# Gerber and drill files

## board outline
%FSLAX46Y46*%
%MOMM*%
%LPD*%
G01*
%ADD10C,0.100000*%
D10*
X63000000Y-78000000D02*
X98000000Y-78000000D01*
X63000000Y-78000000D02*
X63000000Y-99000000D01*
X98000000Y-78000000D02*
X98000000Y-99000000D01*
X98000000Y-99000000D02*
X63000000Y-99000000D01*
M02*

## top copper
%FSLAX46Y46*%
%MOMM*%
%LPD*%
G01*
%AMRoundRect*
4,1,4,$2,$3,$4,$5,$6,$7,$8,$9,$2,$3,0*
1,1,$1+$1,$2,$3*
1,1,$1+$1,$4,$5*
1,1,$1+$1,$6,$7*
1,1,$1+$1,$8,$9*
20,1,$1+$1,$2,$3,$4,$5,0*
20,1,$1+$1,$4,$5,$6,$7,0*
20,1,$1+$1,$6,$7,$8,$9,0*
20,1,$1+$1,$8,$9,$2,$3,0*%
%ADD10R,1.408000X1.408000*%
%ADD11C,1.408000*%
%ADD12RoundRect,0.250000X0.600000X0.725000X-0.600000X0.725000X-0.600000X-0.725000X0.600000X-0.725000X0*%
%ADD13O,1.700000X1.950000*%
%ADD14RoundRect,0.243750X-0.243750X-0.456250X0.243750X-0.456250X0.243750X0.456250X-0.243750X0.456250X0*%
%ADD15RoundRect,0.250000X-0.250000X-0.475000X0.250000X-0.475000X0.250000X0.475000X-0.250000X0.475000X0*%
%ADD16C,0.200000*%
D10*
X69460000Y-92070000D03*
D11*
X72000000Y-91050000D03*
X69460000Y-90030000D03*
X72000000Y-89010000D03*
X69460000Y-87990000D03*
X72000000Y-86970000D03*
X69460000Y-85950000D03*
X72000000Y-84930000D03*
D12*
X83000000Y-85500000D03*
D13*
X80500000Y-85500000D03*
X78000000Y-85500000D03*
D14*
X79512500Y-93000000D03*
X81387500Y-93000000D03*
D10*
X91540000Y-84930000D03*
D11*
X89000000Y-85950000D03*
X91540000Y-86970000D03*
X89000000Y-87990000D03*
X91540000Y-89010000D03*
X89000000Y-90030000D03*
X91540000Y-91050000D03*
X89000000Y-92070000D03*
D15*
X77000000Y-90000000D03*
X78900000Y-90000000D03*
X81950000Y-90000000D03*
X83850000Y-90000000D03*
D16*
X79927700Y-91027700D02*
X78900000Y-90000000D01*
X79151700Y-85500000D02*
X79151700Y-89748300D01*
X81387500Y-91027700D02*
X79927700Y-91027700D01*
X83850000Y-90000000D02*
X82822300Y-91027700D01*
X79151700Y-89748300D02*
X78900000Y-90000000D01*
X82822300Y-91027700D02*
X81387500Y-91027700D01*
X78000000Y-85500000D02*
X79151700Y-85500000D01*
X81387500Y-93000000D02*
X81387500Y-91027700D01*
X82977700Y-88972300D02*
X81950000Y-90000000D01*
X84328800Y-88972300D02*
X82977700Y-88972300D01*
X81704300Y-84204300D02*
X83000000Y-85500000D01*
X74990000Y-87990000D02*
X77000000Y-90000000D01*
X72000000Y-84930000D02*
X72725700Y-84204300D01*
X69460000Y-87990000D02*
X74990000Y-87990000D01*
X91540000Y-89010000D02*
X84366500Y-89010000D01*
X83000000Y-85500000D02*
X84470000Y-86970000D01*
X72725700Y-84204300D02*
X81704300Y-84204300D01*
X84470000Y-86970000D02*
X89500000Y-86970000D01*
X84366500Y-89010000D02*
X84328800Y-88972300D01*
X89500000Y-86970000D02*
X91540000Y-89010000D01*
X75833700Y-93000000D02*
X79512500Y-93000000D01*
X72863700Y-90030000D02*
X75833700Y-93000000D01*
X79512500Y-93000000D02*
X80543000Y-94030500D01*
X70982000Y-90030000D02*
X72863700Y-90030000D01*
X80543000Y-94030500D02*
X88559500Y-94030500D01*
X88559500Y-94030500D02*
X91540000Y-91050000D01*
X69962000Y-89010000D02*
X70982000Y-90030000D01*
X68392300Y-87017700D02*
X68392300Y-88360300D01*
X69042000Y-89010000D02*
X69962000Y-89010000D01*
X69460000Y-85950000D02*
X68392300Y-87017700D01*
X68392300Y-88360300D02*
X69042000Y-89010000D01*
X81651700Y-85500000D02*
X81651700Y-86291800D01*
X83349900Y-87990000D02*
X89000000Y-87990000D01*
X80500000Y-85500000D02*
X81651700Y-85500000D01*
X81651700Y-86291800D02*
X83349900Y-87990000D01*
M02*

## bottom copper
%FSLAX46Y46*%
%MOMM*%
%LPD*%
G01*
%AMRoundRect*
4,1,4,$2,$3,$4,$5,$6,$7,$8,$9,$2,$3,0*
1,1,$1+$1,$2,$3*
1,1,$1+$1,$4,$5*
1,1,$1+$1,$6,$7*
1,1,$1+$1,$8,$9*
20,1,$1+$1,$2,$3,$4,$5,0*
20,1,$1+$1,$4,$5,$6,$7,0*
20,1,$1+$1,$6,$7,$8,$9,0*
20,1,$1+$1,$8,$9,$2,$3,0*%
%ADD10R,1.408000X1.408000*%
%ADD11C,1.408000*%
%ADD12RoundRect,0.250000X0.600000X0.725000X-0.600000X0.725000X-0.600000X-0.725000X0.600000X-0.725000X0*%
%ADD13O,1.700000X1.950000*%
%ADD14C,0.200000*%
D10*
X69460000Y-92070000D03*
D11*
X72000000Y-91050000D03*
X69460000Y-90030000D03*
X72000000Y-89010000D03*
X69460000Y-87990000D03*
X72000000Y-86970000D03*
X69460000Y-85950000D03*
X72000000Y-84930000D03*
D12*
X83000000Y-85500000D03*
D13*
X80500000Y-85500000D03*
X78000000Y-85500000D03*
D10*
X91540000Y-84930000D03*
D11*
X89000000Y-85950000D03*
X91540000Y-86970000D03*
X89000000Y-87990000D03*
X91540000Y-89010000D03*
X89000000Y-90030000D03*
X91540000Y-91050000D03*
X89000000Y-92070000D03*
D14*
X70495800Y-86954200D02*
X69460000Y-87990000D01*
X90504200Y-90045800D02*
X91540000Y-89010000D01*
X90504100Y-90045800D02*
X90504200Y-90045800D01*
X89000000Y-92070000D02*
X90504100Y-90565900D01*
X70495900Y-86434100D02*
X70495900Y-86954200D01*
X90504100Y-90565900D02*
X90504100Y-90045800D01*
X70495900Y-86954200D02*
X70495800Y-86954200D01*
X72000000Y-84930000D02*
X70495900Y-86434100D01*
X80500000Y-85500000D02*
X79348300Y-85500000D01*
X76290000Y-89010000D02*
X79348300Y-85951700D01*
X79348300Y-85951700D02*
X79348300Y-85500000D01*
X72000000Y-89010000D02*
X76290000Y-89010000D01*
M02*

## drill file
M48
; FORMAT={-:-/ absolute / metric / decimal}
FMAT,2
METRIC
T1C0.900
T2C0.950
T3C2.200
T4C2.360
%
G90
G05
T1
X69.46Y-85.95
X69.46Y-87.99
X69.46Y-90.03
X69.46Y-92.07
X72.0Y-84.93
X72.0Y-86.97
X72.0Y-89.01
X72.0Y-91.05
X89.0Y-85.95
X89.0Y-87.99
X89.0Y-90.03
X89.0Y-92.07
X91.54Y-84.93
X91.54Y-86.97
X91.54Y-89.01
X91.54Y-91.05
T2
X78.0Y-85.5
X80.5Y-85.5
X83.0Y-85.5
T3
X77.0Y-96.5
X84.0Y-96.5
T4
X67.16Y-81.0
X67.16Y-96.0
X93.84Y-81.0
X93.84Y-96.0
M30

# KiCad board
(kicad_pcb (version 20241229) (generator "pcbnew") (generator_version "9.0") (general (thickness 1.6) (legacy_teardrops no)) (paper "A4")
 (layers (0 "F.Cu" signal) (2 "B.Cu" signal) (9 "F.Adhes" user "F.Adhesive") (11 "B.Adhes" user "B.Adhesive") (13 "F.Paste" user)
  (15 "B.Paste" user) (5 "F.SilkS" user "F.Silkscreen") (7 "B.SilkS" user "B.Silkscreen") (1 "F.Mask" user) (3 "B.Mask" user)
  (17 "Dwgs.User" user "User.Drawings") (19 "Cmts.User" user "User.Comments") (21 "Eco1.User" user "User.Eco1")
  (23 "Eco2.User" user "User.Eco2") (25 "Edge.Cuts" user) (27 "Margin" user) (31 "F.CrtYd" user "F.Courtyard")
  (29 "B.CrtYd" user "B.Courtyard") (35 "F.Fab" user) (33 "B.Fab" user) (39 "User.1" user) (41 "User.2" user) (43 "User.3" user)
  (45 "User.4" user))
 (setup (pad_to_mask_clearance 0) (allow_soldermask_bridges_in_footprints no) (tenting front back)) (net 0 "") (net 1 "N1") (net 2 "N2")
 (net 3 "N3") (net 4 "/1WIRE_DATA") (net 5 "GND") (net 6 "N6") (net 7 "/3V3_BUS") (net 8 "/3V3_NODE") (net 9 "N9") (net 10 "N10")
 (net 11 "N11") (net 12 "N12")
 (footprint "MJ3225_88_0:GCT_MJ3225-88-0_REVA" (layer "F.Cu") (at 67.585 88.5 -90)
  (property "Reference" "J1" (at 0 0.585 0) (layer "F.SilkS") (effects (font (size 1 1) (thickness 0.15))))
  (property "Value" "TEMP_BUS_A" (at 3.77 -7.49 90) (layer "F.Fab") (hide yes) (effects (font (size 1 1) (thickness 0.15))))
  (pad "" np_thru_hole circle (at -7.5 0.425 270) (size 2.36 2.36) (drill 2.36) (layers "*.Cu" "*.Mask"))
  (pad "" np_thru_hole circle (at 7.5 0.425 270) (size 2.36 2.36) (drill 2.36) (layers "*.Cu" "*.Mask"))
  (pad "1" thru_hole rect (at 3.57 -1.875 270) (size 1.408 1.408) (drill 0.9) (layers "*.Cu" "*.Mask") (remove_unused_layers no)
   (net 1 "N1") (solder_mask_margin 0.102))
  (pad "2" thru_hole circle (at 2.55 -4.415 270) (size 1.408 1.408) (drill 0.9) (layers "*.Cu" "*.Mask") (remove_unused_layers no)
   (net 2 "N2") (solder_mask_margin 0.102))
  (pad "3" thru_hole circle (at 1.53 -1.875 270) (size 1.408 1.408) (drill 0.9) (layers "*.Cu" "*.Mask") (remove_unused_layers no)
   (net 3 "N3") (solder_mask_margin 0.102))
  (pad "4" thru_hole circle (at 0.51 -4.415 270) (size 1.408 1.408) (drill 0.9) (layers "*.Cu" "*.Mask") (remove_unused_layers no)
   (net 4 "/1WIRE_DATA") (solder_mask_margin 0.102))
  (pad "5" thru_hole circle (at -0.51 -1.875 270) (size 1.408 1.408) (drill 0.9) (layers "*.Cu" "*.Mask") (remove_unused_layers no)
   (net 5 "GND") (solder_mask_margin 0.102))
  (pad "6" thru_hole circle (at -1.53 -4.415 270) (size 1.408 1.408) (drill 0.9) (layers "*.Cu" "*.Mask") (remove_unused_layers no)
   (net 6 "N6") (solder_mask_margin 0.102))
  (pad "7" thru_hole circle (at -2.55 -1.875 270) (size 1.408 1.408) (drill 0.9) (layers "*.Cu" "*.Mask") (remove_unused_layers no)
   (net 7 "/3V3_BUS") (solder_mask_margin 0.102))
  (pad "8" thru_hole circle (at -3.57 -4.415 270) (size 1.408 1.408) (drill 0.9) (layers "*.Cu" "*.Mask") (remove_unused_layers no)
   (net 5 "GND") (solder_mask_margin 0.102)))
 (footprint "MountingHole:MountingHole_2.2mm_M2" (layer "F.Cu") (at 84 96.5)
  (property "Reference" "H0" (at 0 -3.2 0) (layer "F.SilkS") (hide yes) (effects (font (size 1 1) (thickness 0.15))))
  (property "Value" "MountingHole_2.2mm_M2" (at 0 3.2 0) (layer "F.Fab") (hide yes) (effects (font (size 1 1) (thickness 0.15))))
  (pad "" np_thru_hole circle (at 0 0) (size 2.2 2.2) (drill 2.2) (layers "*.Cu" "*.Mask")))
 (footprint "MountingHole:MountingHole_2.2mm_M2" (layer "F.Cu") (at 77 96.5)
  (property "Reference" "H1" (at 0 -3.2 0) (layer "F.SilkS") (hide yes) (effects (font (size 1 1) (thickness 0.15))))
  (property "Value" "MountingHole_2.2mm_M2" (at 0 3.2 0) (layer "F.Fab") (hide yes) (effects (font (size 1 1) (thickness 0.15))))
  (pad "" np_thru_hole circle (at 0 0) (size 2.2 2.2) (drill 2.2) (layers "*.Cu" "*.Mask")))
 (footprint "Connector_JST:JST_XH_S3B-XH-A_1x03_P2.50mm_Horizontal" (layer "F.Cu") (at 83 85.5 180)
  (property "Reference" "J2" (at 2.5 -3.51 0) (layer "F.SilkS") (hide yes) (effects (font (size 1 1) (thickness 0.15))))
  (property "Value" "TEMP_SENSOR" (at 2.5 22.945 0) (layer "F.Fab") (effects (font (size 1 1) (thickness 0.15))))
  (pad "1" thru_hole roundrect (at 0 0 180) (size 1.7 1.95) (drill 0.95) (layers "*.Cu" "*.Mask") (remove_unused_layers no)
   (roundrect_rratio 0.147059) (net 5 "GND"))
  (pad "2" thru_hole oval (at 2.5 0 180) (size 1.7 1.95) (drill 0.95) (layers "*.Cu" "*.Mask") (remove_unused_layers no)
   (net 4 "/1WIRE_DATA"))
  (pad "3" thru_hole oval (at 5 0 180) (size 1.7 1.95) (drill 0.95) (layers "*.Cu" "*.Mask") (remove_unused_layers no) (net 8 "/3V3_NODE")))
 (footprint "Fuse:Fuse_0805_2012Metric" (layer "F.Cu") (at 80.45 93)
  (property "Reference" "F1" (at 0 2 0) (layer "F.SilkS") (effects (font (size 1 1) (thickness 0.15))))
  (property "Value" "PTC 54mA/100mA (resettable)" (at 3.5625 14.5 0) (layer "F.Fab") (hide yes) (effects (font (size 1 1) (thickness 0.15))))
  (pad "1" smd roundrect (at -0.9375 0) (size 0.975 1.4) (layers "F.Cu" "F.Mask" "F.Paste") (roundrect_rratio 0.25) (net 7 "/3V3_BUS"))
  (pad "2" smd roundrect (at 0.9375 0) (size 0.975 1.4) (layers "F.Cu" "F.Mask" "F.Paste") (roundrect_rratio 0.25) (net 8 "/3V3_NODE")))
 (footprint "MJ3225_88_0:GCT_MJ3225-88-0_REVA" (layer "F.Cu") (at 93.415 88.5 90)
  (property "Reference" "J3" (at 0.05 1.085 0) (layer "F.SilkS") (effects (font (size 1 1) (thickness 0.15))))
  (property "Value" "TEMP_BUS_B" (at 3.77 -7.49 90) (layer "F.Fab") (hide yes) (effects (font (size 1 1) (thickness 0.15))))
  (pad "" np_thru_hole circle (at -7.5 0.425 90) (size 2.36 2.36) (drill 2.36) (layers "*.Cu" "*.Mask"))
  (pad "" np_thru_hole circle (at 7.5 0.425 90) (size 2.36 2.36) (drill 2.36) (layers "*.Cu" "*.Mask"))
  (pad "1" thru_hole rect (at 3.57 -1.875 90) (size 1.408 1.408) (drill 0.9) (layers "*.Cu" "*.Mask") (remove_unused_layers no) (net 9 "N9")
   (solder_mask_margin 0.102))
  (pad "2" thru_hole circle (at 2.55 -4.415 90) (size 1.408 1.408) (drill 0.9) (layers "*.Cu" "*.Mask") (remove_unused_layers no)
   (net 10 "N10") (solder_mask_margin 0.102))
  (pad "3" thru_hole circle (at 1.53 -1.875 90) (size 1.408 1.408) (drill 0.9) (layers "*.Cu" "*.Mask") (remove_unused_layers no)
   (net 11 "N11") (solder_mask_margin 0.102))
  (pad "4" thru_hole circle (at 0.51 -4.415 90) (size 1.408 1.408) (drill 0.9) (layers "*.Cu" "*.Mask") (remove_unused_layers no)
   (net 4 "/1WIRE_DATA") (solder_mask_margin 0.102))
  (pad "5" thru_hole circle (at -0.51 -1.875 90) (size 1.408 1.408) (drill 0.9) (layers "*.Cu" "*.Mask") (remove_unused_layers no)
   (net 5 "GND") (solder_mask_margin 0.102))
  (pad "6" thru_hole circle (at -1.53 -4.415 90) (size 1.408 1.408) (drill 0.9) (layers "*.Cu" "*.Mask") (remove_unused_layers no)
   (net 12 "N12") (solder_mask_margin 0.102))
  (pad "7" thru_hole circle (at -2.55 -1.875 90) (size 1.408 1.408) (drill 0.9) (layers "*.Cu" "*.Mask") (remove_unused_layers no)
   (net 7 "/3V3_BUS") (solder_mask_margin 0.102))
  (pad "8" thru_hole circle (at -3.57 -4.415 90) (size 1.408 1.408) (drill 0.9) (layers "*.Cu" "*.Mask") (remove_unused_layers no)
   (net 5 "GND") (solder_mask_margin 0.102)))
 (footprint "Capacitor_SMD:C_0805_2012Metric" (layer "F.Cu") (at 77.95 90)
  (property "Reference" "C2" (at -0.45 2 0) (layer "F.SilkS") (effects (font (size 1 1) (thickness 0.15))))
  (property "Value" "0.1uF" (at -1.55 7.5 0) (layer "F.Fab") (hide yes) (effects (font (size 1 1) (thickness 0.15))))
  (pad "1" smd roundrect (at -0.95 0) (size 1 1.45) (layers "F.Cu" "F.Mask" "F.Paste") (roundrect_rratio 0.25) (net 5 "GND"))
  (pad "2" smd roundrect (at 0.95 0) (size 1 1.45) (layers "F.Cu" "F.Mask" "F.Paste") (roundrect_rratio 0.25) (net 8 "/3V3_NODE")))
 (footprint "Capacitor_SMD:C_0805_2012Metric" (layer "F.Cu") (at 82.9 90)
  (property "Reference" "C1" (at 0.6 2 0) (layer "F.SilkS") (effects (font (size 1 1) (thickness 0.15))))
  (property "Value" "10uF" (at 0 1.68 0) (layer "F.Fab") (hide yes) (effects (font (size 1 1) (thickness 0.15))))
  (pad "1" smd roundrect (at -0.95 0) (size 1 1.45) (layers "F.Cu" "F.Mask" "F.Paste") (roundrect_rratio 0.25) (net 5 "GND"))
  (pad "2" smd roundrect (at 0.95 0) (size 1 1.45) (layers "F.Cu" "F.Mask" "F.Paste") (roundrect_rratio 0.25) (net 8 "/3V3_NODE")))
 (gr_line (start 63 78) (end 98 78) (stroke (width 0.1) (type solid)) (layer "Edge.Cuts"))
 (gr_line (start 63 78) (end 63 99) (stroke (width 0.1) (type solid)) (layer "Edge.Cuts"))
 (gr_line (start 98 78) (end 98 99) (stroke (width 0.1) (type solid)) (layer "Edge.Cuts"))
 (gr_line (start 98 99) (end 63 99) (stroke (width 0.1) (type solid)) (layer "Edge.Cuts"))
 (segment (start 79.9277 91.0277) (end 78.9 90) (width 0.2) (layer "F.Cu") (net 8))
 (segment (start 79.1517 85.5) (end 79.1517 89.7483) (width 0.2) (layer "F.Cu") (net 8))
 (segment (start 81.3875 91.0277) (end 79.9277 91.0277) (width 0.2) (layer "F.Cu") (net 8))
 (segment (start 83.85 90) (end 82.8223 91.0277) (width 0.2) (layer "F.Cu") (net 8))
 (segment (start 79.1517 89.7483) (end 78.9 90) (width 0.2) (layer "F.Cu") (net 8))
 (segment (start 82.8223 91.0277) (end 81.3875 91.0277) (width 0.2) (layer "F.Cu") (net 8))
 (segment (start 78 85.5) (end 79.1517 85.5) (width 0.2) (layer "F.Cu") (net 8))
 (segment (start 81.3875 93) (end 81.3875 91.0277) (width 0.2) (layer "F.Cu") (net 8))
 (segment (start 82.9777 88.9723) (end 81.95 90) (width 0.2) (layer "F.Cu") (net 5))
 (segment (start 84.3288 88.9723) (end 82.9777 88.9723) (width 0.2) (layer "F.Cu") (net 5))
 (segment (start 81.7043 84.2043) (end 83 85.5) (width 0.2) (layer "F.Cu") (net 5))
 (segment (start 74.99 87.99) (end 77 90) (width 0.2) (layer "F.Cu") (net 5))
 (segment (start 72 84.93) (end 72.7257 84.2043) (width 0.2) (layer "F.Cu") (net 5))
 (segment (start 69.46 87.99) (end 74.99 87.99) (width 0.2) (layer "F.Cu") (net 5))
 (segment (start 91.54 89.01) (end 84.3665 89.01) (width 0.2) (layer "F.Cu") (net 5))
 (segment (start 83 85.5) (end 84.47 86.97) (width 0.2) (layer "F.Cu") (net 5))
 (segment (start 72.7257 84.2043) (end 81.7043 84.2043) (width 0.2) (layer "F.Cu") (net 5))
 (segment (start 84.47 86.97) (end 89.5 86.97) (width 0.2) (layer "F.Cu") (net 5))
 (segment (start 84.3665 89.01) (end 84.3288 88.9723) (width 0.2) (layer "F.Cu") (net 5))
 (segment (start 89.5 86.97) (end 91.54 89.01) (width 0.2) (layer "F.Cu") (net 5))
 (segment (start 70.4958 86.9542) (end 69.46 87.99) (width 0.2) (layer "B.Cu") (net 5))
 (segment (start 90.5042 90.0458) (end 91.54 89.01) (width 0.2) (layer "B.Cu") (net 5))
 (segment (start 90.5041 90.0458) (end 90.5042 90.0458) (width 0.2) (layer "B.Cu") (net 5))
 (segment (start 89 92.07) (end 90.5041 90.5659) (width 0.2) (layer "B.Cu") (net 5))
 (segment (start 70.4959 86.4341) (end 70.4959 86.9542) (width 0.2) (layer "B.Cu") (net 5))
 (segment (start 90.5041 90.5659) (end 90.5041 90.0458) (width 0.2) (layer "B.Cu") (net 5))
 (segment (start 70.4959 86.9542) (end 70.4958 86.9542) (width 0.2) (layer "B.Cu") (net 5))
 (segment (start 72 84.93) (end 70.4959 86.4341) (width 0.2) (layer "B.Cu") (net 5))
 (segment (start 75.8337 93) (end 79.5125 93) (width 0.2) (layer "F.Cu") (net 7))
 (segment (start 72.8637 90.03) (end 75.8337 93) (width 0.2) (layer "F.Cu") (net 7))
 (segment (start 79.5125 93) (end 80.543 94.0305) (width 0.2) (layer "F.Cu") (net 7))
 (segment (start 70.982 90.03) (end 72.8637 90.03) (width 0.2) (layer "F.Cu") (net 7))
 (segment (start 80.543 94.0305) (end 88.5595 94.0305) (width 0.2) (layer "F.Cu") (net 7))
 (segment (start 88.5595 94.0305) (end 91.54 91.05) (width 0.2) (layer "F.Cu") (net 7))
 (segment (start 69.962 89.01) (end 70.982 90.03) (width 0.2) (layer "F.Cu") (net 7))
 (segment (start 68.3923 87.0177) (end 68.3923 88.3603) (width 0.2) (layer "F.Cu") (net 7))
 (segment (start 69.042 89.01) (end 69.962 89.01) (width 0.2) (layer "F.Cu") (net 7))
 (segment (start 69.46 85.95) (end 68.3923 87.0177) (width 0.2) (layer "F.Cu") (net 7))
 (segment (start 68.3923 88.3603) (end 69.042 89.01) (width 0.2) (layer "F.Cu") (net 7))
 (segment (start 81.6517 85.5) (end 81.6517 86.2918) (width 0.2) (layer "F.Cu") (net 4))
 (segment (start 83.3499 87.99) (end 89 87.99) (width 0.2) (layer "F.Cu") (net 4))
 (segment (start 80.5 85.5) (end 81.6517 85.5) (width 0.2) (layer "F.Cu") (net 4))
 (segment (start 81.6517 86.2918) (end 83.3499 87.99) (width 0.2) (layer "F.Cu") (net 4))
 (segment (start 80.5 85.5) (end 79.3483 85.5) (width 0.2) (layer "B.Cu") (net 4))
 (segment (start 76.29 89.01) (end 79.3483 85.9517) (width 0.2) (layer "B.Cu") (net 4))
 (segment (start 79.3483 85.9517) (end 79.3483 85.5) (width 0.2) (layer "B.Cu") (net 4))
 (segment (start 72 89.01) (end 76.29 89.01) (width 0.2) (layer "B.Cu") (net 4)))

